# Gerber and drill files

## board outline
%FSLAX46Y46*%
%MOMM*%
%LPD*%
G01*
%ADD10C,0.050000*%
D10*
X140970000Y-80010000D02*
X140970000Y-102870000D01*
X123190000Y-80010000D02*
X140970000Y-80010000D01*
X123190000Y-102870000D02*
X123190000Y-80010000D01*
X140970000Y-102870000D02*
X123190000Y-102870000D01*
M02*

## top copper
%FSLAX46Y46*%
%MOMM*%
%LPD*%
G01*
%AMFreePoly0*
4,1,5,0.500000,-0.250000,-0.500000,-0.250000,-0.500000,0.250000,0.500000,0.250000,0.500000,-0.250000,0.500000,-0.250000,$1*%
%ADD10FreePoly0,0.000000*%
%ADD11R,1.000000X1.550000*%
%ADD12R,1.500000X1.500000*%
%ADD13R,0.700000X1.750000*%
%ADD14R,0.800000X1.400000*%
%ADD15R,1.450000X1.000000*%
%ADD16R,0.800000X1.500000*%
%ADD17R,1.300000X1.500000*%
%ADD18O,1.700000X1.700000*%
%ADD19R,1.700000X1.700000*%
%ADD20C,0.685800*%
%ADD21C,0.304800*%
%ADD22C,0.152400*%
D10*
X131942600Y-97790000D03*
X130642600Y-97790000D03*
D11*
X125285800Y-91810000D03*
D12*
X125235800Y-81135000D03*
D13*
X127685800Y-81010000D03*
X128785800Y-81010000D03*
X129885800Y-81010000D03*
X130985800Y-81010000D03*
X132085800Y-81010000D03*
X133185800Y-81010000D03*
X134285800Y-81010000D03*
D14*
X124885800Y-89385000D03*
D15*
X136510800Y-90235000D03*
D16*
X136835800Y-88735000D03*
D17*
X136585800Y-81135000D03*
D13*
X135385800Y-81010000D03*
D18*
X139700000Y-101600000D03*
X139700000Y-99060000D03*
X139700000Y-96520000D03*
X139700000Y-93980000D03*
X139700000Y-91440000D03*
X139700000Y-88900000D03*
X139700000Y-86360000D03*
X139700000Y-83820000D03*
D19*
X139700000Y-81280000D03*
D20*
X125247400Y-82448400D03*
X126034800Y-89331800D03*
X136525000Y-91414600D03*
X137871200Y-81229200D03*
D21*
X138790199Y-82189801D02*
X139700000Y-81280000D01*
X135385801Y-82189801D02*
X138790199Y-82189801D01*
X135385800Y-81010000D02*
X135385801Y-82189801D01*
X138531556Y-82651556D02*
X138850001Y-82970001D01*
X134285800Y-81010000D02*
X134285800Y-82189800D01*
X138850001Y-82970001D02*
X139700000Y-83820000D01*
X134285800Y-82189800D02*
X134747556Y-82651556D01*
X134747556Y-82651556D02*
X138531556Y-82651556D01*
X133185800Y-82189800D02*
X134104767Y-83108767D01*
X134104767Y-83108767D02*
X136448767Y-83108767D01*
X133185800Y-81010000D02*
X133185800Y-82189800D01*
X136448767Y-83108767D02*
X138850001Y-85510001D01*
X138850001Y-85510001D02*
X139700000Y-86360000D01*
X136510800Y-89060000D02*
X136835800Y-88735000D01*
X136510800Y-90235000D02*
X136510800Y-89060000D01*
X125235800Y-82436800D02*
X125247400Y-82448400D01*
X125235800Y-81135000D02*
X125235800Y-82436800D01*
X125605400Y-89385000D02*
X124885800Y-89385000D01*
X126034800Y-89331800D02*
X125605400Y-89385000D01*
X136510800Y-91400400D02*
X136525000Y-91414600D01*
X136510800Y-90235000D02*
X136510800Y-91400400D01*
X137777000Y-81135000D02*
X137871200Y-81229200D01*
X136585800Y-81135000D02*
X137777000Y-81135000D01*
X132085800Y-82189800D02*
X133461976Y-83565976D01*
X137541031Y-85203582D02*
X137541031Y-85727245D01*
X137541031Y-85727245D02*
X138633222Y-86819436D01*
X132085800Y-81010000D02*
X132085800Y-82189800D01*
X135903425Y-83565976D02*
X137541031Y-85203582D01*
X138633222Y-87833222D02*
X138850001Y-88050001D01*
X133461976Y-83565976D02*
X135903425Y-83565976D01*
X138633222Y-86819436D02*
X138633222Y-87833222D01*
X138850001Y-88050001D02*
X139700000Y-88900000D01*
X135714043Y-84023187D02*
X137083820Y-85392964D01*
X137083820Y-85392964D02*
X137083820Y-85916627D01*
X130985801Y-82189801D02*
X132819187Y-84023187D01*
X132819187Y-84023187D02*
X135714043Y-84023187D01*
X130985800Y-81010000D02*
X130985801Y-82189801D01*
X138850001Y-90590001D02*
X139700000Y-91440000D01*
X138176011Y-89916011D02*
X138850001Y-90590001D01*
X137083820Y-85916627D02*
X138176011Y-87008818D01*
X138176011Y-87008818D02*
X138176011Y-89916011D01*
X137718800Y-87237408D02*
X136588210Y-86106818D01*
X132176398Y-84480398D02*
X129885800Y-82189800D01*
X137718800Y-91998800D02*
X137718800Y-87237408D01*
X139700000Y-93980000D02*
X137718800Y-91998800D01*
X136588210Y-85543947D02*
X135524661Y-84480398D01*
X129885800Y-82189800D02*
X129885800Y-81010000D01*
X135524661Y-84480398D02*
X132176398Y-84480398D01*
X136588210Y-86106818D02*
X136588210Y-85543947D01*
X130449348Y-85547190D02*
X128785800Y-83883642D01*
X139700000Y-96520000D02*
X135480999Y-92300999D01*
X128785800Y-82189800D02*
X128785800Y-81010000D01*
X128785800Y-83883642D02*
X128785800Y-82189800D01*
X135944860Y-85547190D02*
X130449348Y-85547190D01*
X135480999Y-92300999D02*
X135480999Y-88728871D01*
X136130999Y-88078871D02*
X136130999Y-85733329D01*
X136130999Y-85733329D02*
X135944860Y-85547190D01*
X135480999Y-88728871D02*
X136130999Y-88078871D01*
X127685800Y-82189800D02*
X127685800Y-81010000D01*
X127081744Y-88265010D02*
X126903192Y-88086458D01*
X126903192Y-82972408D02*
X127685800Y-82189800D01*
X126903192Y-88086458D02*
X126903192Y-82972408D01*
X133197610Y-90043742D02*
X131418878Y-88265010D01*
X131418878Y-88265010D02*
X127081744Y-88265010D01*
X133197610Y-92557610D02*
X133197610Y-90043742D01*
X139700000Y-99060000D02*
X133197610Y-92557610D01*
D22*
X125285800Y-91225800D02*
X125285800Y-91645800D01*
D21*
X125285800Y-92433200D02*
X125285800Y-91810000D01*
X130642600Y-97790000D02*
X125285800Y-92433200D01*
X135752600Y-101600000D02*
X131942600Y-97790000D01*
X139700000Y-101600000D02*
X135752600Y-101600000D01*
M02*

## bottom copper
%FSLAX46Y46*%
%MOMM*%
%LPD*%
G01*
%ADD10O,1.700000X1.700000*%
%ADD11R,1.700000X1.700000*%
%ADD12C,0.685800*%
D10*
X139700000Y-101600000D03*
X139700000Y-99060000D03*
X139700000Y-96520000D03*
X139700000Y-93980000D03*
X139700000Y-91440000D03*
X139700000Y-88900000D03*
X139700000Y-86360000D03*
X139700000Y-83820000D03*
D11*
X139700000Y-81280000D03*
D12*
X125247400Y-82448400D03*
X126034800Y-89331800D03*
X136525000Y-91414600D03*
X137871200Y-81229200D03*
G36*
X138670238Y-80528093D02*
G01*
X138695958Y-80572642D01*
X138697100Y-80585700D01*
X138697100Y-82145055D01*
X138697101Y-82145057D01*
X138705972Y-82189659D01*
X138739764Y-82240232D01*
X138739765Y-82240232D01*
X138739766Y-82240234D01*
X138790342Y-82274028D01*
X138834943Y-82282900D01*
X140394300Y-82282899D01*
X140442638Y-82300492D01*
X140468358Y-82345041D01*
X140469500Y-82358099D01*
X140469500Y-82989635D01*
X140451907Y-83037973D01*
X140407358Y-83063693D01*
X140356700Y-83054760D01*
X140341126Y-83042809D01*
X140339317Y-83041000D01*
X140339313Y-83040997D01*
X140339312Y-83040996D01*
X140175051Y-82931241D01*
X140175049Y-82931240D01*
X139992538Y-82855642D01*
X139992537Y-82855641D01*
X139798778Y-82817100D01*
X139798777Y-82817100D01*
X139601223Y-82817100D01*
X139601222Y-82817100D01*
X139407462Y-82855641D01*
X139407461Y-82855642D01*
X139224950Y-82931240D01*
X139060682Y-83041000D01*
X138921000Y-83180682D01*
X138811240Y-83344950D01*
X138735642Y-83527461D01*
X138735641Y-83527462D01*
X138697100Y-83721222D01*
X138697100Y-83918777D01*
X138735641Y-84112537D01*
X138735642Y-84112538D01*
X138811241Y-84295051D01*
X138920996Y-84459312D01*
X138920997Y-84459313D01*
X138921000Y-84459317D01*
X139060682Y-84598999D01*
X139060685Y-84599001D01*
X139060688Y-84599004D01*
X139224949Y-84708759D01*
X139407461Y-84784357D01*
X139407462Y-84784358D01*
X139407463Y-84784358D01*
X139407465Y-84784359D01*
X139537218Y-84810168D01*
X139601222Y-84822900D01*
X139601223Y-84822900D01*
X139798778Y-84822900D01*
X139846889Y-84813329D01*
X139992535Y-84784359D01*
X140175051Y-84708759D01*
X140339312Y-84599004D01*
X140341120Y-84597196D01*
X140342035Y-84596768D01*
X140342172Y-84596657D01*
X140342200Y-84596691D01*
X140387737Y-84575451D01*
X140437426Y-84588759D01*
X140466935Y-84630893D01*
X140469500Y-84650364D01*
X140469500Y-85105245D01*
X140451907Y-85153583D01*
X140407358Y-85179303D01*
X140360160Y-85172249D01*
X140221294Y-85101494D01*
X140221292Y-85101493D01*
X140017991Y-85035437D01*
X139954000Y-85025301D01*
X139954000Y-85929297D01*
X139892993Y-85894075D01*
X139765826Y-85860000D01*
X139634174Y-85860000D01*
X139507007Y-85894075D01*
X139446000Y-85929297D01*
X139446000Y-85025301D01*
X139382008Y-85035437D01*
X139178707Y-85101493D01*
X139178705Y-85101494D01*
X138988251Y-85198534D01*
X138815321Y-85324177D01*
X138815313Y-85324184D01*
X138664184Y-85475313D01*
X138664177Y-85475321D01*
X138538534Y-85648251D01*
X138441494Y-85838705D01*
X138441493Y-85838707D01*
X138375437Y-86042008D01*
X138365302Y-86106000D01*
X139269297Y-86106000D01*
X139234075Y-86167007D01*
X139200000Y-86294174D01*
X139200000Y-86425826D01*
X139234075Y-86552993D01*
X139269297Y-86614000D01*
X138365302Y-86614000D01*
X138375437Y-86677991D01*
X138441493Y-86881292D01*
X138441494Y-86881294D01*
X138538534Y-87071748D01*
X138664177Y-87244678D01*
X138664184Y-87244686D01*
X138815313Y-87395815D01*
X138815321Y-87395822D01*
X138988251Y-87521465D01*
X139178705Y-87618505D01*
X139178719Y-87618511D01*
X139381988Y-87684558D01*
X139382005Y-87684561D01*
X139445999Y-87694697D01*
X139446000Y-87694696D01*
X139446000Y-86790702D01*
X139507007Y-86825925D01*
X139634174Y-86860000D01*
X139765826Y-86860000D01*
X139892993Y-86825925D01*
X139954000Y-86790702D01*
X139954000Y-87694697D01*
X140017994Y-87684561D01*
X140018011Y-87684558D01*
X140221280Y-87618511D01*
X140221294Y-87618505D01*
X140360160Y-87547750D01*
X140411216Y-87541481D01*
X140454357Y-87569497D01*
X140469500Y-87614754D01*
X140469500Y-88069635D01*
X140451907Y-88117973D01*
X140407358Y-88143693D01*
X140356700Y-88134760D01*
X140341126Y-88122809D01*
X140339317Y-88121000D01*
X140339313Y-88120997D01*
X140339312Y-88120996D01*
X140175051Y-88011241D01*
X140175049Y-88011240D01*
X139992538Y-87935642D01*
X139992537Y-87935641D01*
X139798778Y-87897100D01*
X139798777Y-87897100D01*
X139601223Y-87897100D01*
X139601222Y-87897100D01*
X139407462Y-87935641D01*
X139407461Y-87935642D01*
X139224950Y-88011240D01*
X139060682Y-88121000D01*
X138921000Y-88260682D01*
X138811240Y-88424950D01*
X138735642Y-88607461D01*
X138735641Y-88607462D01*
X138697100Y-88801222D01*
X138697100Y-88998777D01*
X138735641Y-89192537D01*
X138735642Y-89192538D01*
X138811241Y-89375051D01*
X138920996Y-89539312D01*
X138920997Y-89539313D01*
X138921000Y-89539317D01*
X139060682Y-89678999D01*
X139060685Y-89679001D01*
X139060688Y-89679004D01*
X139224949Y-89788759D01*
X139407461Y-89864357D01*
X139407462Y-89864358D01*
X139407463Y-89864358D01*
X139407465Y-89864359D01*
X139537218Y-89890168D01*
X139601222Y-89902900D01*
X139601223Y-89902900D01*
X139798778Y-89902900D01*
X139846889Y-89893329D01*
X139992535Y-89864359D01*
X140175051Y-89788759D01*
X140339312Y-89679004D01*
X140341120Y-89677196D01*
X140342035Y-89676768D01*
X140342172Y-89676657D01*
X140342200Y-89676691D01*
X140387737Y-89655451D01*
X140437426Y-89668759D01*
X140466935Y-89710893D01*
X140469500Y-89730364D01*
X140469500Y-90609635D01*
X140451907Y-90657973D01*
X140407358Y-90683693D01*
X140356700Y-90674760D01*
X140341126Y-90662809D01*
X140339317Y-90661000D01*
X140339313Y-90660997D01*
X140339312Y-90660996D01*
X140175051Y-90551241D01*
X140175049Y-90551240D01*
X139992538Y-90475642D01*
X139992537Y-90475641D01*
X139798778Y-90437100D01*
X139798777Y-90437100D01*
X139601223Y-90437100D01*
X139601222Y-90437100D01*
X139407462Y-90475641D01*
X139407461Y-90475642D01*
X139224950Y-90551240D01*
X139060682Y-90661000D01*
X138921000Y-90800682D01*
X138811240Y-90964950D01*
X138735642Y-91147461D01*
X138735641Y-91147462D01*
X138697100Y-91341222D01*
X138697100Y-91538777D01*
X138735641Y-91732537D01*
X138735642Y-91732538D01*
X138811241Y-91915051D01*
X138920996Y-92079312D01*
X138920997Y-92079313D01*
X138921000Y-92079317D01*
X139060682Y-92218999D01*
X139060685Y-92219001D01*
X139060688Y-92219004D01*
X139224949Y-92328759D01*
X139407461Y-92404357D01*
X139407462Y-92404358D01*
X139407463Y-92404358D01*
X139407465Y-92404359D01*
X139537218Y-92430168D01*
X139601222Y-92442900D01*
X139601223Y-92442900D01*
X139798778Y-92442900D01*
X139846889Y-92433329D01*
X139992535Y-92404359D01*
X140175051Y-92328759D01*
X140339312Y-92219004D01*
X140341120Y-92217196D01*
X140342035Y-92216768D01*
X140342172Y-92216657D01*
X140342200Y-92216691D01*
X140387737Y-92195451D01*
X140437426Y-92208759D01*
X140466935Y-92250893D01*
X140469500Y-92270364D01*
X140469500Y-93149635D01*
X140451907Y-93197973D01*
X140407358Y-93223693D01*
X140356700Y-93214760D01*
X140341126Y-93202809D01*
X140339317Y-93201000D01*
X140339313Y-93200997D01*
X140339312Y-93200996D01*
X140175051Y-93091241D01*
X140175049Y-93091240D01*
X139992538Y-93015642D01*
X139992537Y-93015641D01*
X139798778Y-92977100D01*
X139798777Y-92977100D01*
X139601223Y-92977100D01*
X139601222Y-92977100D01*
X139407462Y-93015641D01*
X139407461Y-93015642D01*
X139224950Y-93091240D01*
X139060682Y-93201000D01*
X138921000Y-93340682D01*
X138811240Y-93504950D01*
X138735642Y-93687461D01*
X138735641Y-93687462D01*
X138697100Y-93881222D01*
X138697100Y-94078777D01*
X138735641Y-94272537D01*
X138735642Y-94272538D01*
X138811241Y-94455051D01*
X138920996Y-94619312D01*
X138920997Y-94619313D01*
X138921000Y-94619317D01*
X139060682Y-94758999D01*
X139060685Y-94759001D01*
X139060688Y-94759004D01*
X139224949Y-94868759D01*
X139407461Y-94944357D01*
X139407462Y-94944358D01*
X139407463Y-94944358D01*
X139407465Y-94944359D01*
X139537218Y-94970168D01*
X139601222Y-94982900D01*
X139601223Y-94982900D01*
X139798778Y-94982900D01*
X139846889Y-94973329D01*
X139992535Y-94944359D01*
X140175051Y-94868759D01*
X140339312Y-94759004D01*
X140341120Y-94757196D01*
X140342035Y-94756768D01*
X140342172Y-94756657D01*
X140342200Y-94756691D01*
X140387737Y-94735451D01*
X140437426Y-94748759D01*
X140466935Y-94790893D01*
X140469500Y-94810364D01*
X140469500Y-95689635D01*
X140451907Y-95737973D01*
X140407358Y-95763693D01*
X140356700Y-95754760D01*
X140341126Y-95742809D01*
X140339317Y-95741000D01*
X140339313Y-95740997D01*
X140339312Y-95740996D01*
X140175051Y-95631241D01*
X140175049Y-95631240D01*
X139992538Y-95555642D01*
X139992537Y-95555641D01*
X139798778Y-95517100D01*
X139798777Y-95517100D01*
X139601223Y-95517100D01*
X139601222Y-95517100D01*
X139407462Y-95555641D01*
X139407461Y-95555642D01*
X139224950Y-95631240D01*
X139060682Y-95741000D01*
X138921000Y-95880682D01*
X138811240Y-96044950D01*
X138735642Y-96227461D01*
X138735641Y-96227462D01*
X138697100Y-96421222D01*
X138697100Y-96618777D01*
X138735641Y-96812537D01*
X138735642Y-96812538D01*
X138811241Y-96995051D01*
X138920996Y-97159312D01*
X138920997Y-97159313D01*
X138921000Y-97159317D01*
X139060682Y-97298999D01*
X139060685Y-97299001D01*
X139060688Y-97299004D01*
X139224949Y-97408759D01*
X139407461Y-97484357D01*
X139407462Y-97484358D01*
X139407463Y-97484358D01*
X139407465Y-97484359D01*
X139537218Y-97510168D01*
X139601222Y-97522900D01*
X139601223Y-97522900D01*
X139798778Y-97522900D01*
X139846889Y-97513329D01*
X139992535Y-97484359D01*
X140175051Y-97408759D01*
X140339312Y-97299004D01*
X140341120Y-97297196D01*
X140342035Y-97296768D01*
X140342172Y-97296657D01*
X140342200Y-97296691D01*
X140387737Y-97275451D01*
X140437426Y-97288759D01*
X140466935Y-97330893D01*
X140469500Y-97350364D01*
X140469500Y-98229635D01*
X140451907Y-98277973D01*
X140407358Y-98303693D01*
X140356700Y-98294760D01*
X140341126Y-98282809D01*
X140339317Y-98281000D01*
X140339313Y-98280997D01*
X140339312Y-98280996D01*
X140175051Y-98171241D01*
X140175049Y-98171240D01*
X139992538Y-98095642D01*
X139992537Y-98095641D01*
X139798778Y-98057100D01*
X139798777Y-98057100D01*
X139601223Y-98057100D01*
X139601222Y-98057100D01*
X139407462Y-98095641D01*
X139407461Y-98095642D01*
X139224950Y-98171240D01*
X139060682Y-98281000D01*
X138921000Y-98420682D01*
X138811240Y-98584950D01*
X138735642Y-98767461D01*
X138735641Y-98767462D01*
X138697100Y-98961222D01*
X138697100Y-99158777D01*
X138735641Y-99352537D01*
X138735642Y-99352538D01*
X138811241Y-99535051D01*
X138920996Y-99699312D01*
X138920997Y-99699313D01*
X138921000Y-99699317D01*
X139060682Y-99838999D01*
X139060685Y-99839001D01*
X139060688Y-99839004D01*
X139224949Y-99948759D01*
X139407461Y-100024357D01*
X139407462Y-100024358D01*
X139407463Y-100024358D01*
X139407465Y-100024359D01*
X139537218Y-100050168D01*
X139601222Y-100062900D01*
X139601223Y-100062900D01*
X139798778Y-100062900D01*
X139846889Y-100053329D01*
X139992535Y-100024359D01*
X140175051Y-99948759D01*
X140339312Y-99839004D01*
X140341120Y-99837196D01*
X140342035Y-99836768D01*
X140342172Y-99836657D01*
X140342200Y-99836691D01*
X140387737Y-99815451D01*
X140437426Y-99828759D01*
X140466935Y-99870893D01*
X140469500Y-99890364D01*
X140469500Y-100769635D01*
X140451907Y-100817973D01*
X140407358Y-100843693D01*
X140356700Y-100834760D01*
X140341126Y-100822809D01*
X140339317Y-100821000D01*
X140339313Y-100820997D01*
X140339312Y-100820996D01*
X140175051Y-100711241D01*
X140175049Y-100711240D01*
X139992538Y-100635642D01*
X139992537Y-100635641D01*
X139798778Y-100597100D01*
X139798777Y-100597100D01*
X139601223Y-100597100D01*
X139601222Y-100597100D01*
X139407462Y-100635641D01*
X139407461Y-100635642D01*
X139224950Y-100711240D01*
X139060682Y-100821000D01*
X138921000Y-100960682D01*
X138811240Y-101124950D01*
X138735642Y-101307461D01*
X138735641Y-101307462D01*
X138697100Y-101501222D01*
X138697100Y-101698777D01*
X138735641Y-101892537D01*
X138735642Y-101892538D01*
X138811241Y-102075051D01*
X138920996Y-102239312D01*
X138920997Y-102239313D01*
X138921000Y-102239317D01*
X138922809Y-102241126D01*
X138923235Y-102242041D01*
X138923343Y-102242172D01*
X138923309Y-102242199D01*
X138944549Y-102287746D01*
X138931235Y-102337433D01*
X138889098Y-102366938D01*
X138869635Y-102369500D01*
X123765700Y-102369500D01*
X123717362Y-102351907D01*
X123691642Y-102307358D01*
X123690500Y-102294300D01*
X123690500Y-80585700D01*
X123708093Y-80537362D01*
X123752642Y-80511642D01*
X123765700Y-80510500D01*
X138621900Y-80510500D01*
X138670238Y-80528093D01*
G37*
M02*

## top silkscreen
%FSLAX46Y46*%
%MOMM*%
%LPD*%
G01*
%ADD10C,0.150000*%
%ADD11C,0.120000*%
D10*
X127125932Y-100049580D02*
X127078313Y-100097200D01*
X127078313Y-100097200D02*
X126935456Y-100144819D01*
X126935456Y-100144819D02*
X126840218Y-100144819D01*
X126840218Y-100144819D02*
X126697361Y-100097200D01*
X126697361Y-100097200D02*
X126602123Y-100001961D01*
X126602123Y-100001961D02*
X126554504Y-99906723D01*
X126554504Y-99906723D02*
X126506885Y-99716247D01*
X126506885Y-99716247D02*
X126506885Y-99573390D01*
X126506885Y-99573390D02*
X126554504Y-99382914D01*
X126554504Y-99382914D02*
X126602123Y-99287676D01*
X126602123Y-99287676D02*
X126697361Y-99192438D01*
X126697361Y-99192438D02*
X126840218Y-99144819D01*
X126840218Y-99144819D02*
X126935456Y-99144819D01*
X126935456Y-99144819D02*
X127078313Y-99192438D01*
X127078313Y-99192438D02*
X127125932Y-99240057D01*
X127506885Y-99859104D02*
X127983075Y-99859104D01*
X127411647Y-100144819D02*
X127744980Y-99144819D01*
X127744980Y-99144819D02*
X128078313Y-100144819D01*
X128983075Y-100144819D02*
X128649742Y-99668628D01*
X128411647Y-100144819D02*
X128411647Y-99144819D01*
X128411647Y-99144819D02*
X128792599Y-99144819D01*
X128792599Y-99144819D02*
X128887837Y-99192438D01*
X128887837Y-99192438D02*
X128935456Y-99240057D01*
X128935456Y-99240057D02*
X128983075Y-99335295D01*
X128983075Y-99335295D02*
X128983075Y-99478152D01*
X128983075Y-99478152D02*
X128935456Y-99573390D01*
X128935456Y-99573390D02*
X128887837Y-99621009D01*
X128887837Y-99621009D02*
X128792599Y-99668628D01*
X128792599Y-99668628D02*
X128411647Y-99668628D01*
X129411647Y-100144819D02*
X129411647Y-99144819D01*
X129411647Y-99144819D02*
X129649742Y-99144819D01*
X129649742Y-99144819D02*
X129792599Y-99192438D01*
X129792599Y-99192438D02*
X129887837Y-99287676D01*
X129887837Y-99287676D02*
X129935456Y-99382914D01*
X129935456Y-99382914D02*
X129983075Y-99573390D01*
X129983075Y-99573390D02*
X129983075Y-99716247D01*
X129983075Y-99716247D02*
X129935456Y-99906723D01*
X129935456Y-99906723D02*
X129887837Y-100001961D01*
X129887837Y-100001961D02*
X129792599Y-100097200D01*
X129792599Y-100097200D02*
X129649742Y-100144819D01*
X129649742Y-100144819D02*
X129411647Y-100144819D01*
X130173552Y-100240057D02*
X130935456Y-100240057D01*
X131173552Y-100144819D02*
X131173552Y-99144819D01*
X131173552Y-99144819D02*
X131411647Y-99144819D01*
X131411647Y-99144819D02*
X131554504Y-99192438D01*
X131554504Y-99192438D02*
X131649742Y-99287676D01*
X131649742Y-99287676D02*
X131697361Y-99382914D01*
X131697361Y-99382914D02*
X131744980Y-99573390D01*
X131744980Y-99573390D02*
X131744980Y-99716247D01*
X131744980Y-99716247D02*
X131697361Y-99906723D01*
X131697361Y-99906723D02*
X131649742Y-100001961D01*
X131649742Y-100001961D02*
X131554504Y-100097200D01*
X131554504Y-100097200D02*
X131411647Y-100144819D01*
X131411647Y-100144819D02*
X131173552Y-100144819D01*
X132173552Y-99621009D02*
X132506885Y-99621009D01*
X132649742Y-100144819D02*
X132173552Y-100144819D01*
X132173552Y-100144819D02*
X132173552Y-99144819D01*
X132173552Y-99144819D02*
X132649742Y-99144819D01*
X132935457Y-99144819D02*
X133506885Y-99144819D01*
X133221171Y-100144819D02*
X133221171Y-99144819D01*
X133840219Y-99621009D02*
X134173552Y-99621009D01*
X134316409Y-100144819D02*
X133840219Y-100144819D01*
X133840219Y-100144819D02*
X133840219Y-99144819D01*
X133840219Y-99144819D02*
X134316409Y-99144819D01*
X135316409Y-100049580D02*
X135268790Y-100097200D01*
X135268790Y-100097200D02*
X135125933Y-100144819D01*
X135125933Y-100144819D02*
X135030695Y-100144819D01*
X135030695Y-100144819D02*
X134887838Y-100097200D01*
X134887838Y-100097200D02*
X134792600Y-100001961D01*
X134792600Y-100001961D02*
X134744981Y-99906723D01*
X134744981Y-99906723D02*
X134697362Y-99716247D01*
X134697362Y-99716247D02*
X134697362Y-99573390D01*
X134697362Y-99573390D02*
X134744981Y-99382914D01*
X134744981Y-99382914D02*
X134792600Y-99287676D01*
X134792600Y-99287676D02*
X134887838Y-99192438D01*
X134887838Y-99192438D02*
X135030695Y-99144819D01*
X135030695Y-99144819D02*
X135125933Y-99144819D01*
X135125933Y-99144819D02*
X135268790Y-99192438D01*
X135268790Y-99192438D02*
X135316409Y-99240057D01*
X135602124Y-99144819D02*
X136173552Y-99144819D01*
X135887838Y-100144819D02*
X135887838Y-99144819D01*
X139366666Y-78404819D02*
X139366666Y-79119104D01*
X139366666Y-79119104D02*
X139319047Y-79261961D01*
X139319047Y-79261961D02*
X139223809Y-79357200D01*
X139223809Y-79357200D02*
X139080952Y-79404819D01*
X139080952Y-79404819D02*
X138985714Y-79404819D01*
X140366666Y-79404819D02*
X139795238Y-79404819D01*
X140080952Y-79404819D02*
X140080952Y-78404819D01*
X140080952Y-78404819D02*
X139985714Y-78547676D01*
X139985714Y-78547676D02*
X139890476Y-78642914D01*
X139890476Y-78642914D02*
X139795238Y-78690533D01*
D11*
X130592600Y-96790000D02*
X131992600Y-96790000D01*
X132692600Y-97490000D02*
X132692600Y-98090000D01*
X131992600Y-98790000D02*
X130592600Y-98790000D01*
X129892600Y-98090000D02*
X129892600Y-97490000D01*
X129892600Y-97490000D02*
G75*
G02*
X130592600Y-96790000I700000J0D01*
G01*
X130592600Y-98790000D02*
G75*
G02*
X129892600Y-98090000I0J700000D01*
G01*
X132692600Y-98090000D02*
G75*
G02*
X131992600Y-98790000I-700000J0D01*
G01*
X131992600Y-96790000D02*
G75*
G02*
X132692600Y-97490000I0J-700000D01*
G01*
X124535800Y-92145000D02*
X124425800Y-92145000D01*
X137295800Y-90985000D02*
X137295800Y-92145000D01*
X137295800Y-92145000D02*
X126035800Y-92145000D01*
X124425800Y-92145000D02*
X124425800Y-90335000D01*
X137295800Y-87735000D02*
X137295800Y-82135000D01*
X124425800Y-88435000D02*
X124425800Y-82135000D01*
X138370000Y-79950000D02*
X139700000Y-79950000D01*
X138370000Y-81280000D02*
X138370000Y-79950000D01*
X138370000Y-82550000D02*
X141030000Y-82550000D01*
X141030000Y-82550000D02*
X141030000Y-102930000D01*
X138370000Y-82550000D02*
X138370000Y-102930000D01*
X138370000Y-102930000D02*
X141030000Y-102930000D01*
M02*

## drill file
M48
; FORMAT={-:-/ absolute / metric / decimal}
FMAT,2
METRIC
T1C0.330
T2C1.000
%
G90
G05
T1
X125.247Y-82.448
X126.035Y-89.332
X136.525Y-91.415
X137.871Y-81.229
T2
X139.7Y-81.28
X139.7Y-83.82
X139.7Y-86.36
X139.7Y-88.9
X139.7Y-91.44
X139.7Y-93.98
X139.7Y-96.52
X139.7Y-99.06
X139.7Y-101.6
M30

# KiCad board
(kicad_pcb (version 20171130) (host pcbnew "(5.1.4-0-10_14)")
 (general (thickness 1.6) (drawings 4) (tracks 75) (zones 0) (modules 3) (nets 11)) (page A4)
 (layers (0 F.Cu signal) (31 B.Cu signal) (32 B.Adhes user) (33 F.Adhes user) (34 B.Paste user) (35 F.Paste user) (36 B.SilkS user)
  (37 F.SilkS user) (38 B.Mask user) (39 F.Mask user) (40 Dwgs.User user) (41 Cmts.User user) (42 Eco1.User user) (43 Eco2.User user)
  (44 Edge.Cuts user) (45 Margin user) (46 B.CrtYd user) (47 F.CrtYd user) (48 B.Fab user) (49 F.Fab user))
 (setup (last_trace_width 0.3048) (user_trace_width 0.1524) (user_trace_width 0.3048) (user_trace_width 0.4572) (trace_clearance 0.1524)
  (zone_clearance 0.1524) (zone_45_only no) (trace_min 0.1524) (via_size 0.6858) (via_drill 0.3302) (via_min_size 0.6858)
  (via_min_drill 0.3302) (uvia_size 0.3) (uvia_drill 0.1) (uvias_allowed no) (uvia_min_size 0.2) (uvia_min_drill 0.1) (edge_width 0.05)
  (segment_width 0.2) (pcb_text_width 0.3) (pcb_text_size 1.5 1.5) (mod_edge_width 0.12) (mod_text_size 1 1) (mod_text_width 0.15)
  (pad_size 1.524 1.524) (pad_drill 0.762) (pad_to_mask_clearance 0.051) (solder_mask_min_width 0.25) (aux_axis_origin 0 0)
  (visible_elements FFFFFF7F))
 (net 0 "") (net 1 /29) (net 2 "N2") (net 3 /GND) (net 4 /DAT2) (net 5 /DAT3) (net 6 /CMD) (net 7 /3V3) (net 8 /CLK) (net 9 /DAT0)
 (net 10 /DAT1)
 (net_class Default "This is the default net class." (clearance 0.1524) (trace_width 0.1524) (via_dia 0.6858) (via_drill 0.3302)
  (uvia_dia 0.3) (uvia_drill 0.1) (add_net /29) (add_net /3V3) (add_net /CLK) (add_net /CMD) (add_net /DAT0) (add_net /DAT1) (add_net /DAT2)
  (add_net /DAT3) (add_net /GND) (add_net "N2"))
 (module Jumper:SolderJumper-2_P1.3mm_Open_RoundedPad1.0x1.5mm (layer F.Cu) (at 131.2926 97.79)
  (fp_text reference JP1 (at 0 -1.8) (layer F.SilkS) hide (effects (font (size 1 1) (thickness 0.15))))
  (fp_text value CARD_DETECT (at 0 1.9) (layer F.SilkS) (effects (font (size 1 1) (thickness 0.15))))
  (fp_line (start -0.7 -1) (end 0.7 -1) (layer F.SilkS) (width 0.12))
  (fp_line (start 1.4 -0.3) (end 1.4 0.3) (layer F.SilkS) (width 0.12))
  (fp_line (start 0.7 1) (end -0.7 1) (layer F.SilkS) (width 0.12))
  (fp_line (start -1.4 0.3) (end -1.4 -0.3) (layer F.SilkS) (width 0.12))
  (fp_arc (start -0.7 -0.3) (end -0.7 -1) (angle -90) (layer F.SilkS) (width 0.12))
  (fp_arc (start -0.7 0.3) (end -1.4 0.3) (angle -90) (layer F.SilkS) (width 0.12))
  (fp_arc (start 0.7 0.3) (end 0.7 1) (angle -90) (layer F.SilkS) (width 0.12))
  (fp_arc (start 0.7 -0.3) (end 1.4 -0.3) (angle -90) (layer F.SilkS) (width 0.12))
  (pad 2 smd custom (at 0.65 0) (size 1 0.5) (layers F.Cu F.Mask) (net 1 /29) (zone_connect 2) (options (clearance outline) (anchor rect))
   (primitives))
  (pad 1 smd custom (at -0.65 0) (size 1 0.5) (layers F.Cu F.Mask) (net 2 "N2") (zone_connect 2) (options (clearance outline) (anchor rect))
   (primitives)))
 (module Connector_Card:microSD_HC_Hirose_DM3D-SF (layer F.Cu) (at 130.8608 86.36 180)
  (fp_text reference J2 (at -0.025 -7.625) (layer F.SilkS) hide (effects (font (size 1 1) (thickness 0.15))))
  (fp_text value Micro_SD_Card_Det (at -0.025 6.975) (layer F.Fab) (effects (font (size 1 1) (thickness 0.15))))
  (fp_line (start 6.325 -5.785) (end 6.435 -5.785) (layer F.SilkS) (width 0.12))
  (fp_line (start -6.435 -4.625) (end -6.435 -5.785) (layer F.SilkS) (width 0.12))
  (fp_line (start -6.435 -5.785) (end 4.825 -5.785) (layer F.SilkS) (width 0.12))
  (fp_line (start 6.435 -5.785) (end 6.435 -3.975) (layer F.SilkS) (width 0.12))
  (fp_line (start -6.435 -1.375) (end -6.435 4.225) (layer F.SilkS) (width 0.12))
  (fp_line (start 6.435 -2.075) (end 6.435 4.225) (layer F.SilkS) (width 0.12))
  (pad 10 smd rect (at 5.575 -5.45 180) (size 1 1.55) (layers F.Cu F.Paste F.Mask) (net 2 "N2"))
  (pad 11 smd rect (at 5.625 5.225 180) (size 1.5 1.5) (layers F.Cu F.Paste F.Mask) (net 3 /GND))
  (pad 1 smd rect (at 3.175 5.35 180) (size 0.7 1.75) (layers F.Cu F.Paste F.Mask) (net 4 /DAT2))
  (pad 2 smd rect (at 2.075 5.35 180) (size 0.7 1.75) (layers F.Cu F.Paste F.Mask) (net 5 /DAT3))
  (pad 3 smd rect (at 0.975 5.35 180) (size 0.7 1.75) (layers F.Cu F.Paste F.Mask) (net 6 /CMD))
  (pad 4 smd rect (at -0.125 5.35 180) (size 0.7 1.75) (layers F.Cu F.Paste F.Mask) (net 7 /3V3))
  (pad 5 smd rect (at -1.225 5.35 180) (size 0.7 1.75) (layers F.Cu F.Paste F.Mask) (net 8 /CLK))
  (pad 6 smd rect (at -2.325 5.35 180) (size 0.7 1.75) (layers F.Cu F.Paste F.Mask) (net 3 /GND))
  (pad 7 smd rect (at -3.425 5.35 180) (size 0.7 1.75) (layers F.Cu F.Paste F.Mask) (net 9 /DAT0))
  (pad 11 smd rect (at 5.975 -3.025 180) (size 0.8 1.4) (layers F.Cu F.Paste F.Mask) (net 3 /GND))
  (pad 9 smd rect (at -5.65 -3.875 180) (size 1.45 1) (layers F.Cu F.Paste F.Mask) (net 3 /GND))
  (pad 11 smd rect (at -5.975 -2.375 180) (size 0.8 1.5) (layers F.Cu F.Paste F.Mask) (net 3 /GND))
  (pad 11 smd rect (at -5.725 5.225 180) (size 1.3 1.5) (layers F.Cu F.Paste F.Mask) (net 3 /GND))
  (pad 8 smd rect (at -4.525 5.35 180) (size 0.7 1.75) (layers F.Cu F.Paste F.Mask) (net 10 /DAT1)))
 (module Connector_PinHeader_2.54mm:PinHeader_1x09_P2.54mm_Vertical (layer F.Cu) (at 139.7 81.28)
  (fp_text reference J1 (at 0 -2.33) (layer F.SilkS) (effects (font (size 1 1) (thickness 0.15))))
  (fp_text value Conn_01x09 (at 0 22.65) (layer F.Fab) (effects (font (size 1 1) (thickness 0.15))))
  (fp_line (start -1.33 -1.33) (end 0 -1.33) (layer F.SilkS) (width 0.12))
  (fp_line (start -1.33 0) (end -1.33 -1.33) (layer F.SilkS) (width 0.12))
  (fp_line (start -1.33 1.27) (end 1.33 1.27) (layer F.SilkS) (width 0.12))
  (fp_line (start 1.33 1.27) (end 1.33 21.65) (layer F.SilkS) (width 0.12))
  (fp_line (start -1.33 1.27) (end -1.33 21.65) (layer F.SilkS) (width 0.12))
  (fp_line (start -1.33 21.65) (end 1.33 21.65) (layer F.SilkS) (width 0.12))
  (pad 9 thru_hole oval (at 0 20.32) (size 1.7 1.7) (drill 1) (layers *.Cu *.Mask) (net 1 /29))
  (pad 8 thru_hole oval (at 0 17.78) (size 1.7 1.7) (drill 1) (layers *.Cu *.Mask) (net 4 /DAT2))
  (pad 7 thru_hole oval (at 0 15.24) (size 1.7 1.7) (drill 1) (layers *.Cu *.Mask) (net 5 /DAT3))
  (pad 6 thru_hole oval (at 0 12.7) (size 1.7 1.7) (drill 1) (layers *.Cu *.Mask) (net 6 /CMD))
  (pad 5 thru_hole oval (at 0 10.16) (size 1.7 1.7) (drill 1) (layers *.Cu *.Mask) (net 7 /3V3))
  (pad 4 thru_hole oval (at 0 7.62) (size 1.7 1.7) (drill 1) (layers *.Cu *.Mask) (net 8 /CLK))
  (pad 3 thru_hole oval (at 0 5.08) (size 1.7 1.7) (drill 1) (layers *.Cu *.Mask) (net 3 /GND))
  (pad 2 thru_hole oval (at 0 2.54) (size 1.7 1.7) (drill 1) (layers *.Cu *.Mask) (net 9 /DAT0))
  (pad 1 thru_hole rect (at 0 0) (size 1.7 1.7) (drill 1) (layers *.Cu *.Mask) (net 10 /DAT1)))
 (gr_line (start 140.97 80.01) (end 140.97 102.87) (layer Edge.Cuts) (width 0.05))
 (gr_line (start 123.19 80.01) (end 140.97 80.01) (layer Edge.Cuts) (width 0.05))
 (gr_line (start 123.19 102.87) (end 123.19 80.01) (layer Edge.Cuts) (width 0.05))
 (gr_line (start 140.97 102.87) (end 123.19 102.87) (layer Edge.Cuts) (width 0.05))
 (segment (start 138.790199 82.189801) (end 139.7 81.28) (width 0.3048) (layer F.Cu) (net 10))
 (segment (start 135.385801 82.189801) (end 138.790199 82.189801) (width 0.3048) (layer F.Cu) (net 10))
 (segment (start 135.3858 81.01) (end 135.385801 82.189801) (width 0.3048) (layer F.Cu) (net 10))
 (segment (start 138.531556 82.651556) (end 138.850001 82.970001) (width 0.3048) (layer F.Cu) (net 9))
 (segment (start 134.2858 81.01) (end 134.2858 82.1898) (width 0.3048) (layer F.Cu) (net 9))
 (segment (start 138.850001 82.970001) (end 139.7 83.82) (width 0.3048) (layer F.Cu) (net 9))
 (segment (start 134.2858 82.1898) (end 134.747556 82.651556) (width 0.3048) (layer F.Cu) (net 9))
 (segment (start 134.747556 82.651556) (end 138.531556 82.651556) (width 0.3048) (layer F.Cu) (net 9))
 (segment (start 133.1858 82.1898) (end 134.104767 83.108767) (width 0.3048) (layer F.Cu) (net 3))
 (segment (start 134.104767 83.108767) (end 136.448767 83.108767) (width 0.3048) (layer F.Cu) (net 3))
 (segment (start 133.1858 81.01) (end 133.1858 82.1898) (width 0.3048) (layer F.Cu) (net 3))
 (segment (start 136.448767 83.108767) (end 138.850001 85.510001) (width 0.3048) (layer F.Cu) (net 3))
 (segment (start 138.850001 85.510001) (end 139.7 86.36) (width 0.3048) (layer F.Cu) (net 3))
 (segment (start 136.5108 89.06) (end 136.8358 88.735) (width 0.3048) (layer F.Cu) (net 3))
 (segment (start 136.5108 90.235) (end 136.5108 89.06) (width 0.3048) (layer F.Cu) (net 3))
 (segment (start 125.2358 82.4368) (end 125.2474 82.4484) (width 0.3048) (layer F.Cu) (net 3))
 (via (at 125.2474 82.4484) (size 0.6858) (drill 0.3302) (layers F.Cu B.Cu) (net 3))
 (segment (start 125.2358 81.135) (end 125.2358 82.4368) (width 0.3048) (layer F.Cu) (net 3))
 (segment (start 125.6054 89.385) (end 124.8858 89.385) (width 0.3048) (layer F.Cu) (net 3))
 (segment (start 126.0348 89.3318) (end 125.6054 89.385) (width 0.3048) (layer F.Cu) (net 3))
 (via (at 126.0348 89.3318) (size 0.6858) (drill 0.3302) (layers F.Cu B.Cu) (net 3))
 (via (at 136.525 91.4146) (size 0.6858) (drill 0.3302) (layers F.Cu B.Cu) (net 3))
 (segment (start 136.5108 91.4004) (end 136.525 91.4146) (width 0.3048) (layer F.Cu) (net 3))
 (segment (start 136.5108 90.235) (end 136.5108 91.4004) (width 0.3048) (layer F.Cu) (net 3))
 (via (at 137.8712 81.2292) (size 0.6858) (drill 0.3302) (layers F.Cu B.Cu) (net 3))
 (segment (start 137.777 81.135) (end 137.8712 81.2292) (width 0.3048) (layer F.Cu) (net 3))
 (segment (start 136.5858 81.135) (end 137.777 81.135) (width 0.3048) (layer F.Cu) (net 3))
 (segment (start 132.0858 82.1898) (end 133.461976 83.565976) (width 0.3048) (layer F.Cu) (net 8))
 (segment (start 137.541031 85.203582) (end 137.541031 85.727245) (width 0.3048) (layer F.Cu) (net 8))
 (segment (start 137.541031 85.727245) (end 138.633222 86.819436) (width 0.3048) (layer F.Cu) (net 8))
 (segment (start 132.0858 81.01) (end 132.0858 82.1898) (width 0.3048) (layer F.Cu) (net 8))
 (segment (start 135.903425 83.565976) (end 137.541031 85.203582) (width 0.3048) (layer F.Cu) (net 8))
 (segment (start 138.633222 87.833222) (end 138.850001 88.050001) (width 0.3048) (layer F.Cu) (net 8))
 (segment (start 133.461976 83.565976) (end 135.903425 83.565976) (width 0.3048) (layer F.Cu) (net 8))
 (segment (start 138.633222 86.819436) (end 138.633222 87.833222) (width 0.3048) (layer F.Cu) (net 8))
 (segment (start 138.850001 88.050001) (end 139.7 88.9) (width 0.3048) (layer F.Cu) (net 8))
 (segment (start 135.714043 84.023187) (end 137.08382 85.392964) (width 0.3048) (layer F.Cu) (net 7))
 (segment (start 137.08382 85.392964) (end 137.08382 85.916627) (width 0.3048) (layer F.Cu) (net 7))
 (segment (start 130.985801 82.189801) (end 132.819187 84.023187) (width 0.3048) (layer F.Cu) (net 7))
 (segment (start 132.819187 84.023187) (end 135.714043 84.023187) (width 0.3048) (layer F.Cu) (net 7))
 (segment (start 130.9858 81.01) (end 130.985801 82.189801) (width 0.3048) (layer F.Cu) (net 7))
 (segment (start 138.850001 90.590001) (end 139.7 91.44) (width 0.3048) (layer F.Cu) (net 7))
 (segment (start 138.176011 89.916011) (end 138.850001 90.590001) (width 0.3048) (layer F.Cu) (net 7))
 (segment (start 137.08382 85.916627) (end 138.176011 87.008818) (width 0.3048) (layer F.Cu) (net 7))
 (segment (start 138.176011 87.008818) (end 138.176011 89.916011) (width 0.3048) (layer F.Cu) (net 7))
 (segment (start 137.7188 87.237408) (end 136.58821 86.106818) (width 0.3048) (layer F.Cu) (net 6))
 (segment (start 132.176398 84.480398) (end 129.8858 82.1898) (width 0.3048) (layer F.Cu) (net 6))
 (segment (start 137.7188 91.9988) (end 137.7188 87.237408) (width 0.3048) (layer F.Cu) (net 6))
 (segment (start 139.7 93.98) (end 137.7188 91.9988) (width 0.3048) (layer F.Cu) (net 6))
 (segment (start 136.58821 85.543947) (end 135.524661 84.480398) (width 0.3048) (layer F.Cu) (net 6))
 (segment (start 129.8858 82.1898) (end 129.8858 81.01) (width 0.3048) (layer F.Cu) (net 6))
 (segment (start 135.524661 84.480398) (end 132.176398 84.480398) (width 0.3048) (layer F.Cu) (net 6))
 (segment (start 136.58821 86.106818) (end 136.58821 85.543947) (width 0.3048) (layer F.Cu) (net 6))
 (segment (start 130.449348 85.54719) (end 128.7858 83.883642) (width 0.3048) (layer F.Cu) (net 5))
 (segment (start 139.7 96.52) (end 135.480999 92.300999) (width 0.3048) (layer F.Cu) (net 5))
 (segment (start 128.7858 82.1898) (end 128.7858 81.01) (width 0.3048) (layer F.Cu) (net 5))
 (segment (start 128.7858 83.883642) (end 128.7858 82.1898) (width 0.3048) (layer F.Cu) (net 5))
 (segment (start 135.94486 85.54719) (end 130.449348 85.54719) (width 0.3048) (layer F.Cu) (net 5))
 (segment (start 135.480999 92.300999) (end 135.480999 88.728871) (width 0.3048) (layer F.Cu) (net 5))
 (segment (start 136.130999 88.078871) (end 136.130999 85.733329) (width 0.3048) (layer F.Cu) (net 5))
 (segment (start 136.130999 85.733329) (end 135.94486 85.54719) (width 0.3048) (layer F.Cu) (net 5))
 (segment (start 135.480999 88.728871) (end 136.130999 88.078871) (width 0.3048) (layer F.Cu) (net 5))
 (segment (start 127.6858 82.1898) (end 127.6858 81.01) (width 0.3048) (layer F.Cu) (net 4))
 (segment (start 127.081744 88.26501) (end 126.903192 88.086458) (width 0.3048) (layer F.Cu) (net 4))
 (segment (start 126.903192 82.972408) (end 127.6858 82.1898) (width 0.3048) (layer F.Cu) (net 4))
 (segment (start 126.903192 88.086458) (end 126.903192 82.972408) (width 0.3048) (layer F.Cu) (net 4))
 (segment (start 133.19761 90.043742) (end 131.418878 88.26501) (width 0.3048) (layer F.Cu) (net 4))
 (segment (start 131.418878 88.26501) (end 127.081744 88.26501) (width 0.3048) (layer F.Cu) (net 4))
 (segment (start 133.19761 92.55761) (end 133.19761 90.043742) (width 0.3048) (layer F.Cu) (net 4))
 (segment (start 139.7 99.06) (end 133.19761 92.55761) (width 0.3048) (layer F.Cu) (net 4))
 (segment (start 125.2858 91.2258) (end 125.2858 91.6458) (width 0.1524) (layer F.Cu) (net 2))
 (segment (start 125.2858 92.4332) (end 125.2858 91.81) (width 0.3048) (layer F.Cu) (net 2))
 (segment (start 130.6426 97.79) (end 125.2858 92.4332) (width 0.3048) (layer F.Cu) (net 2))
 (segment (start 135.7526 101.6) (end 131.9426 97.79) (width 0.3048) (layer F.Cu) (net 1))
 (segment (start 139.7 101.6) (end 135.7526 101.6) (width 0.3048) (layer F.Cu) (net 1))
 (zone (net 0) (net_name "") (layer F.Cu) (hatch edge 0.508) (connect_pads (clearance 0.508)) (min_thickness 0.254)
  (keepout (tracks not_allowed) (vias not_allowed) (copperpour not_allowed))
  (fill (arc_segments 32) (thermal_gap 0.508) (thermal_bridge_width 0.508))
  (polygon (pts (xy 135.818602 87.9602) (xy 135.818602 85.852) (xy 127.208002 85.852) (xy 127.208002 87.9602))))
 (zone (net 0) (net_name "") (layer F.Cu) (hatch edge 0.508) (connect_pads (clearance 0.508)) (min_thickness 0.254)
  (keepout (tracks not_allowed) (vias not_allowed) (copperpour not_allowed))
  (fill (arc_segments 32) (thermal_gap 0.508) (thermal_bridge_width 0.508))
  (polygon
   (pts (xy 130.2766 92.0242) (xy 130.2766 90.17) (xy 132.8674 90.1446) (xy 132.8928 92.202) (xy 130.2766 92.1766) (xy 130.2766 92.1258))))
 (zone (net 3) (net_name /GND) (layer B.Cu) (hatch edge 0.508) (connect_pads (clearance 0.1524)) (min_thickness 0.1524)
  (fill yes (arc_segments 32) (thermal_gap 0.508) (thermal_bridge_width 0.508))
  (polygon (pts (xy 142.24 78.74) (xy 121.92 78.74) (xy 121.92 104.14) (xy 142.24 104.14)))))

